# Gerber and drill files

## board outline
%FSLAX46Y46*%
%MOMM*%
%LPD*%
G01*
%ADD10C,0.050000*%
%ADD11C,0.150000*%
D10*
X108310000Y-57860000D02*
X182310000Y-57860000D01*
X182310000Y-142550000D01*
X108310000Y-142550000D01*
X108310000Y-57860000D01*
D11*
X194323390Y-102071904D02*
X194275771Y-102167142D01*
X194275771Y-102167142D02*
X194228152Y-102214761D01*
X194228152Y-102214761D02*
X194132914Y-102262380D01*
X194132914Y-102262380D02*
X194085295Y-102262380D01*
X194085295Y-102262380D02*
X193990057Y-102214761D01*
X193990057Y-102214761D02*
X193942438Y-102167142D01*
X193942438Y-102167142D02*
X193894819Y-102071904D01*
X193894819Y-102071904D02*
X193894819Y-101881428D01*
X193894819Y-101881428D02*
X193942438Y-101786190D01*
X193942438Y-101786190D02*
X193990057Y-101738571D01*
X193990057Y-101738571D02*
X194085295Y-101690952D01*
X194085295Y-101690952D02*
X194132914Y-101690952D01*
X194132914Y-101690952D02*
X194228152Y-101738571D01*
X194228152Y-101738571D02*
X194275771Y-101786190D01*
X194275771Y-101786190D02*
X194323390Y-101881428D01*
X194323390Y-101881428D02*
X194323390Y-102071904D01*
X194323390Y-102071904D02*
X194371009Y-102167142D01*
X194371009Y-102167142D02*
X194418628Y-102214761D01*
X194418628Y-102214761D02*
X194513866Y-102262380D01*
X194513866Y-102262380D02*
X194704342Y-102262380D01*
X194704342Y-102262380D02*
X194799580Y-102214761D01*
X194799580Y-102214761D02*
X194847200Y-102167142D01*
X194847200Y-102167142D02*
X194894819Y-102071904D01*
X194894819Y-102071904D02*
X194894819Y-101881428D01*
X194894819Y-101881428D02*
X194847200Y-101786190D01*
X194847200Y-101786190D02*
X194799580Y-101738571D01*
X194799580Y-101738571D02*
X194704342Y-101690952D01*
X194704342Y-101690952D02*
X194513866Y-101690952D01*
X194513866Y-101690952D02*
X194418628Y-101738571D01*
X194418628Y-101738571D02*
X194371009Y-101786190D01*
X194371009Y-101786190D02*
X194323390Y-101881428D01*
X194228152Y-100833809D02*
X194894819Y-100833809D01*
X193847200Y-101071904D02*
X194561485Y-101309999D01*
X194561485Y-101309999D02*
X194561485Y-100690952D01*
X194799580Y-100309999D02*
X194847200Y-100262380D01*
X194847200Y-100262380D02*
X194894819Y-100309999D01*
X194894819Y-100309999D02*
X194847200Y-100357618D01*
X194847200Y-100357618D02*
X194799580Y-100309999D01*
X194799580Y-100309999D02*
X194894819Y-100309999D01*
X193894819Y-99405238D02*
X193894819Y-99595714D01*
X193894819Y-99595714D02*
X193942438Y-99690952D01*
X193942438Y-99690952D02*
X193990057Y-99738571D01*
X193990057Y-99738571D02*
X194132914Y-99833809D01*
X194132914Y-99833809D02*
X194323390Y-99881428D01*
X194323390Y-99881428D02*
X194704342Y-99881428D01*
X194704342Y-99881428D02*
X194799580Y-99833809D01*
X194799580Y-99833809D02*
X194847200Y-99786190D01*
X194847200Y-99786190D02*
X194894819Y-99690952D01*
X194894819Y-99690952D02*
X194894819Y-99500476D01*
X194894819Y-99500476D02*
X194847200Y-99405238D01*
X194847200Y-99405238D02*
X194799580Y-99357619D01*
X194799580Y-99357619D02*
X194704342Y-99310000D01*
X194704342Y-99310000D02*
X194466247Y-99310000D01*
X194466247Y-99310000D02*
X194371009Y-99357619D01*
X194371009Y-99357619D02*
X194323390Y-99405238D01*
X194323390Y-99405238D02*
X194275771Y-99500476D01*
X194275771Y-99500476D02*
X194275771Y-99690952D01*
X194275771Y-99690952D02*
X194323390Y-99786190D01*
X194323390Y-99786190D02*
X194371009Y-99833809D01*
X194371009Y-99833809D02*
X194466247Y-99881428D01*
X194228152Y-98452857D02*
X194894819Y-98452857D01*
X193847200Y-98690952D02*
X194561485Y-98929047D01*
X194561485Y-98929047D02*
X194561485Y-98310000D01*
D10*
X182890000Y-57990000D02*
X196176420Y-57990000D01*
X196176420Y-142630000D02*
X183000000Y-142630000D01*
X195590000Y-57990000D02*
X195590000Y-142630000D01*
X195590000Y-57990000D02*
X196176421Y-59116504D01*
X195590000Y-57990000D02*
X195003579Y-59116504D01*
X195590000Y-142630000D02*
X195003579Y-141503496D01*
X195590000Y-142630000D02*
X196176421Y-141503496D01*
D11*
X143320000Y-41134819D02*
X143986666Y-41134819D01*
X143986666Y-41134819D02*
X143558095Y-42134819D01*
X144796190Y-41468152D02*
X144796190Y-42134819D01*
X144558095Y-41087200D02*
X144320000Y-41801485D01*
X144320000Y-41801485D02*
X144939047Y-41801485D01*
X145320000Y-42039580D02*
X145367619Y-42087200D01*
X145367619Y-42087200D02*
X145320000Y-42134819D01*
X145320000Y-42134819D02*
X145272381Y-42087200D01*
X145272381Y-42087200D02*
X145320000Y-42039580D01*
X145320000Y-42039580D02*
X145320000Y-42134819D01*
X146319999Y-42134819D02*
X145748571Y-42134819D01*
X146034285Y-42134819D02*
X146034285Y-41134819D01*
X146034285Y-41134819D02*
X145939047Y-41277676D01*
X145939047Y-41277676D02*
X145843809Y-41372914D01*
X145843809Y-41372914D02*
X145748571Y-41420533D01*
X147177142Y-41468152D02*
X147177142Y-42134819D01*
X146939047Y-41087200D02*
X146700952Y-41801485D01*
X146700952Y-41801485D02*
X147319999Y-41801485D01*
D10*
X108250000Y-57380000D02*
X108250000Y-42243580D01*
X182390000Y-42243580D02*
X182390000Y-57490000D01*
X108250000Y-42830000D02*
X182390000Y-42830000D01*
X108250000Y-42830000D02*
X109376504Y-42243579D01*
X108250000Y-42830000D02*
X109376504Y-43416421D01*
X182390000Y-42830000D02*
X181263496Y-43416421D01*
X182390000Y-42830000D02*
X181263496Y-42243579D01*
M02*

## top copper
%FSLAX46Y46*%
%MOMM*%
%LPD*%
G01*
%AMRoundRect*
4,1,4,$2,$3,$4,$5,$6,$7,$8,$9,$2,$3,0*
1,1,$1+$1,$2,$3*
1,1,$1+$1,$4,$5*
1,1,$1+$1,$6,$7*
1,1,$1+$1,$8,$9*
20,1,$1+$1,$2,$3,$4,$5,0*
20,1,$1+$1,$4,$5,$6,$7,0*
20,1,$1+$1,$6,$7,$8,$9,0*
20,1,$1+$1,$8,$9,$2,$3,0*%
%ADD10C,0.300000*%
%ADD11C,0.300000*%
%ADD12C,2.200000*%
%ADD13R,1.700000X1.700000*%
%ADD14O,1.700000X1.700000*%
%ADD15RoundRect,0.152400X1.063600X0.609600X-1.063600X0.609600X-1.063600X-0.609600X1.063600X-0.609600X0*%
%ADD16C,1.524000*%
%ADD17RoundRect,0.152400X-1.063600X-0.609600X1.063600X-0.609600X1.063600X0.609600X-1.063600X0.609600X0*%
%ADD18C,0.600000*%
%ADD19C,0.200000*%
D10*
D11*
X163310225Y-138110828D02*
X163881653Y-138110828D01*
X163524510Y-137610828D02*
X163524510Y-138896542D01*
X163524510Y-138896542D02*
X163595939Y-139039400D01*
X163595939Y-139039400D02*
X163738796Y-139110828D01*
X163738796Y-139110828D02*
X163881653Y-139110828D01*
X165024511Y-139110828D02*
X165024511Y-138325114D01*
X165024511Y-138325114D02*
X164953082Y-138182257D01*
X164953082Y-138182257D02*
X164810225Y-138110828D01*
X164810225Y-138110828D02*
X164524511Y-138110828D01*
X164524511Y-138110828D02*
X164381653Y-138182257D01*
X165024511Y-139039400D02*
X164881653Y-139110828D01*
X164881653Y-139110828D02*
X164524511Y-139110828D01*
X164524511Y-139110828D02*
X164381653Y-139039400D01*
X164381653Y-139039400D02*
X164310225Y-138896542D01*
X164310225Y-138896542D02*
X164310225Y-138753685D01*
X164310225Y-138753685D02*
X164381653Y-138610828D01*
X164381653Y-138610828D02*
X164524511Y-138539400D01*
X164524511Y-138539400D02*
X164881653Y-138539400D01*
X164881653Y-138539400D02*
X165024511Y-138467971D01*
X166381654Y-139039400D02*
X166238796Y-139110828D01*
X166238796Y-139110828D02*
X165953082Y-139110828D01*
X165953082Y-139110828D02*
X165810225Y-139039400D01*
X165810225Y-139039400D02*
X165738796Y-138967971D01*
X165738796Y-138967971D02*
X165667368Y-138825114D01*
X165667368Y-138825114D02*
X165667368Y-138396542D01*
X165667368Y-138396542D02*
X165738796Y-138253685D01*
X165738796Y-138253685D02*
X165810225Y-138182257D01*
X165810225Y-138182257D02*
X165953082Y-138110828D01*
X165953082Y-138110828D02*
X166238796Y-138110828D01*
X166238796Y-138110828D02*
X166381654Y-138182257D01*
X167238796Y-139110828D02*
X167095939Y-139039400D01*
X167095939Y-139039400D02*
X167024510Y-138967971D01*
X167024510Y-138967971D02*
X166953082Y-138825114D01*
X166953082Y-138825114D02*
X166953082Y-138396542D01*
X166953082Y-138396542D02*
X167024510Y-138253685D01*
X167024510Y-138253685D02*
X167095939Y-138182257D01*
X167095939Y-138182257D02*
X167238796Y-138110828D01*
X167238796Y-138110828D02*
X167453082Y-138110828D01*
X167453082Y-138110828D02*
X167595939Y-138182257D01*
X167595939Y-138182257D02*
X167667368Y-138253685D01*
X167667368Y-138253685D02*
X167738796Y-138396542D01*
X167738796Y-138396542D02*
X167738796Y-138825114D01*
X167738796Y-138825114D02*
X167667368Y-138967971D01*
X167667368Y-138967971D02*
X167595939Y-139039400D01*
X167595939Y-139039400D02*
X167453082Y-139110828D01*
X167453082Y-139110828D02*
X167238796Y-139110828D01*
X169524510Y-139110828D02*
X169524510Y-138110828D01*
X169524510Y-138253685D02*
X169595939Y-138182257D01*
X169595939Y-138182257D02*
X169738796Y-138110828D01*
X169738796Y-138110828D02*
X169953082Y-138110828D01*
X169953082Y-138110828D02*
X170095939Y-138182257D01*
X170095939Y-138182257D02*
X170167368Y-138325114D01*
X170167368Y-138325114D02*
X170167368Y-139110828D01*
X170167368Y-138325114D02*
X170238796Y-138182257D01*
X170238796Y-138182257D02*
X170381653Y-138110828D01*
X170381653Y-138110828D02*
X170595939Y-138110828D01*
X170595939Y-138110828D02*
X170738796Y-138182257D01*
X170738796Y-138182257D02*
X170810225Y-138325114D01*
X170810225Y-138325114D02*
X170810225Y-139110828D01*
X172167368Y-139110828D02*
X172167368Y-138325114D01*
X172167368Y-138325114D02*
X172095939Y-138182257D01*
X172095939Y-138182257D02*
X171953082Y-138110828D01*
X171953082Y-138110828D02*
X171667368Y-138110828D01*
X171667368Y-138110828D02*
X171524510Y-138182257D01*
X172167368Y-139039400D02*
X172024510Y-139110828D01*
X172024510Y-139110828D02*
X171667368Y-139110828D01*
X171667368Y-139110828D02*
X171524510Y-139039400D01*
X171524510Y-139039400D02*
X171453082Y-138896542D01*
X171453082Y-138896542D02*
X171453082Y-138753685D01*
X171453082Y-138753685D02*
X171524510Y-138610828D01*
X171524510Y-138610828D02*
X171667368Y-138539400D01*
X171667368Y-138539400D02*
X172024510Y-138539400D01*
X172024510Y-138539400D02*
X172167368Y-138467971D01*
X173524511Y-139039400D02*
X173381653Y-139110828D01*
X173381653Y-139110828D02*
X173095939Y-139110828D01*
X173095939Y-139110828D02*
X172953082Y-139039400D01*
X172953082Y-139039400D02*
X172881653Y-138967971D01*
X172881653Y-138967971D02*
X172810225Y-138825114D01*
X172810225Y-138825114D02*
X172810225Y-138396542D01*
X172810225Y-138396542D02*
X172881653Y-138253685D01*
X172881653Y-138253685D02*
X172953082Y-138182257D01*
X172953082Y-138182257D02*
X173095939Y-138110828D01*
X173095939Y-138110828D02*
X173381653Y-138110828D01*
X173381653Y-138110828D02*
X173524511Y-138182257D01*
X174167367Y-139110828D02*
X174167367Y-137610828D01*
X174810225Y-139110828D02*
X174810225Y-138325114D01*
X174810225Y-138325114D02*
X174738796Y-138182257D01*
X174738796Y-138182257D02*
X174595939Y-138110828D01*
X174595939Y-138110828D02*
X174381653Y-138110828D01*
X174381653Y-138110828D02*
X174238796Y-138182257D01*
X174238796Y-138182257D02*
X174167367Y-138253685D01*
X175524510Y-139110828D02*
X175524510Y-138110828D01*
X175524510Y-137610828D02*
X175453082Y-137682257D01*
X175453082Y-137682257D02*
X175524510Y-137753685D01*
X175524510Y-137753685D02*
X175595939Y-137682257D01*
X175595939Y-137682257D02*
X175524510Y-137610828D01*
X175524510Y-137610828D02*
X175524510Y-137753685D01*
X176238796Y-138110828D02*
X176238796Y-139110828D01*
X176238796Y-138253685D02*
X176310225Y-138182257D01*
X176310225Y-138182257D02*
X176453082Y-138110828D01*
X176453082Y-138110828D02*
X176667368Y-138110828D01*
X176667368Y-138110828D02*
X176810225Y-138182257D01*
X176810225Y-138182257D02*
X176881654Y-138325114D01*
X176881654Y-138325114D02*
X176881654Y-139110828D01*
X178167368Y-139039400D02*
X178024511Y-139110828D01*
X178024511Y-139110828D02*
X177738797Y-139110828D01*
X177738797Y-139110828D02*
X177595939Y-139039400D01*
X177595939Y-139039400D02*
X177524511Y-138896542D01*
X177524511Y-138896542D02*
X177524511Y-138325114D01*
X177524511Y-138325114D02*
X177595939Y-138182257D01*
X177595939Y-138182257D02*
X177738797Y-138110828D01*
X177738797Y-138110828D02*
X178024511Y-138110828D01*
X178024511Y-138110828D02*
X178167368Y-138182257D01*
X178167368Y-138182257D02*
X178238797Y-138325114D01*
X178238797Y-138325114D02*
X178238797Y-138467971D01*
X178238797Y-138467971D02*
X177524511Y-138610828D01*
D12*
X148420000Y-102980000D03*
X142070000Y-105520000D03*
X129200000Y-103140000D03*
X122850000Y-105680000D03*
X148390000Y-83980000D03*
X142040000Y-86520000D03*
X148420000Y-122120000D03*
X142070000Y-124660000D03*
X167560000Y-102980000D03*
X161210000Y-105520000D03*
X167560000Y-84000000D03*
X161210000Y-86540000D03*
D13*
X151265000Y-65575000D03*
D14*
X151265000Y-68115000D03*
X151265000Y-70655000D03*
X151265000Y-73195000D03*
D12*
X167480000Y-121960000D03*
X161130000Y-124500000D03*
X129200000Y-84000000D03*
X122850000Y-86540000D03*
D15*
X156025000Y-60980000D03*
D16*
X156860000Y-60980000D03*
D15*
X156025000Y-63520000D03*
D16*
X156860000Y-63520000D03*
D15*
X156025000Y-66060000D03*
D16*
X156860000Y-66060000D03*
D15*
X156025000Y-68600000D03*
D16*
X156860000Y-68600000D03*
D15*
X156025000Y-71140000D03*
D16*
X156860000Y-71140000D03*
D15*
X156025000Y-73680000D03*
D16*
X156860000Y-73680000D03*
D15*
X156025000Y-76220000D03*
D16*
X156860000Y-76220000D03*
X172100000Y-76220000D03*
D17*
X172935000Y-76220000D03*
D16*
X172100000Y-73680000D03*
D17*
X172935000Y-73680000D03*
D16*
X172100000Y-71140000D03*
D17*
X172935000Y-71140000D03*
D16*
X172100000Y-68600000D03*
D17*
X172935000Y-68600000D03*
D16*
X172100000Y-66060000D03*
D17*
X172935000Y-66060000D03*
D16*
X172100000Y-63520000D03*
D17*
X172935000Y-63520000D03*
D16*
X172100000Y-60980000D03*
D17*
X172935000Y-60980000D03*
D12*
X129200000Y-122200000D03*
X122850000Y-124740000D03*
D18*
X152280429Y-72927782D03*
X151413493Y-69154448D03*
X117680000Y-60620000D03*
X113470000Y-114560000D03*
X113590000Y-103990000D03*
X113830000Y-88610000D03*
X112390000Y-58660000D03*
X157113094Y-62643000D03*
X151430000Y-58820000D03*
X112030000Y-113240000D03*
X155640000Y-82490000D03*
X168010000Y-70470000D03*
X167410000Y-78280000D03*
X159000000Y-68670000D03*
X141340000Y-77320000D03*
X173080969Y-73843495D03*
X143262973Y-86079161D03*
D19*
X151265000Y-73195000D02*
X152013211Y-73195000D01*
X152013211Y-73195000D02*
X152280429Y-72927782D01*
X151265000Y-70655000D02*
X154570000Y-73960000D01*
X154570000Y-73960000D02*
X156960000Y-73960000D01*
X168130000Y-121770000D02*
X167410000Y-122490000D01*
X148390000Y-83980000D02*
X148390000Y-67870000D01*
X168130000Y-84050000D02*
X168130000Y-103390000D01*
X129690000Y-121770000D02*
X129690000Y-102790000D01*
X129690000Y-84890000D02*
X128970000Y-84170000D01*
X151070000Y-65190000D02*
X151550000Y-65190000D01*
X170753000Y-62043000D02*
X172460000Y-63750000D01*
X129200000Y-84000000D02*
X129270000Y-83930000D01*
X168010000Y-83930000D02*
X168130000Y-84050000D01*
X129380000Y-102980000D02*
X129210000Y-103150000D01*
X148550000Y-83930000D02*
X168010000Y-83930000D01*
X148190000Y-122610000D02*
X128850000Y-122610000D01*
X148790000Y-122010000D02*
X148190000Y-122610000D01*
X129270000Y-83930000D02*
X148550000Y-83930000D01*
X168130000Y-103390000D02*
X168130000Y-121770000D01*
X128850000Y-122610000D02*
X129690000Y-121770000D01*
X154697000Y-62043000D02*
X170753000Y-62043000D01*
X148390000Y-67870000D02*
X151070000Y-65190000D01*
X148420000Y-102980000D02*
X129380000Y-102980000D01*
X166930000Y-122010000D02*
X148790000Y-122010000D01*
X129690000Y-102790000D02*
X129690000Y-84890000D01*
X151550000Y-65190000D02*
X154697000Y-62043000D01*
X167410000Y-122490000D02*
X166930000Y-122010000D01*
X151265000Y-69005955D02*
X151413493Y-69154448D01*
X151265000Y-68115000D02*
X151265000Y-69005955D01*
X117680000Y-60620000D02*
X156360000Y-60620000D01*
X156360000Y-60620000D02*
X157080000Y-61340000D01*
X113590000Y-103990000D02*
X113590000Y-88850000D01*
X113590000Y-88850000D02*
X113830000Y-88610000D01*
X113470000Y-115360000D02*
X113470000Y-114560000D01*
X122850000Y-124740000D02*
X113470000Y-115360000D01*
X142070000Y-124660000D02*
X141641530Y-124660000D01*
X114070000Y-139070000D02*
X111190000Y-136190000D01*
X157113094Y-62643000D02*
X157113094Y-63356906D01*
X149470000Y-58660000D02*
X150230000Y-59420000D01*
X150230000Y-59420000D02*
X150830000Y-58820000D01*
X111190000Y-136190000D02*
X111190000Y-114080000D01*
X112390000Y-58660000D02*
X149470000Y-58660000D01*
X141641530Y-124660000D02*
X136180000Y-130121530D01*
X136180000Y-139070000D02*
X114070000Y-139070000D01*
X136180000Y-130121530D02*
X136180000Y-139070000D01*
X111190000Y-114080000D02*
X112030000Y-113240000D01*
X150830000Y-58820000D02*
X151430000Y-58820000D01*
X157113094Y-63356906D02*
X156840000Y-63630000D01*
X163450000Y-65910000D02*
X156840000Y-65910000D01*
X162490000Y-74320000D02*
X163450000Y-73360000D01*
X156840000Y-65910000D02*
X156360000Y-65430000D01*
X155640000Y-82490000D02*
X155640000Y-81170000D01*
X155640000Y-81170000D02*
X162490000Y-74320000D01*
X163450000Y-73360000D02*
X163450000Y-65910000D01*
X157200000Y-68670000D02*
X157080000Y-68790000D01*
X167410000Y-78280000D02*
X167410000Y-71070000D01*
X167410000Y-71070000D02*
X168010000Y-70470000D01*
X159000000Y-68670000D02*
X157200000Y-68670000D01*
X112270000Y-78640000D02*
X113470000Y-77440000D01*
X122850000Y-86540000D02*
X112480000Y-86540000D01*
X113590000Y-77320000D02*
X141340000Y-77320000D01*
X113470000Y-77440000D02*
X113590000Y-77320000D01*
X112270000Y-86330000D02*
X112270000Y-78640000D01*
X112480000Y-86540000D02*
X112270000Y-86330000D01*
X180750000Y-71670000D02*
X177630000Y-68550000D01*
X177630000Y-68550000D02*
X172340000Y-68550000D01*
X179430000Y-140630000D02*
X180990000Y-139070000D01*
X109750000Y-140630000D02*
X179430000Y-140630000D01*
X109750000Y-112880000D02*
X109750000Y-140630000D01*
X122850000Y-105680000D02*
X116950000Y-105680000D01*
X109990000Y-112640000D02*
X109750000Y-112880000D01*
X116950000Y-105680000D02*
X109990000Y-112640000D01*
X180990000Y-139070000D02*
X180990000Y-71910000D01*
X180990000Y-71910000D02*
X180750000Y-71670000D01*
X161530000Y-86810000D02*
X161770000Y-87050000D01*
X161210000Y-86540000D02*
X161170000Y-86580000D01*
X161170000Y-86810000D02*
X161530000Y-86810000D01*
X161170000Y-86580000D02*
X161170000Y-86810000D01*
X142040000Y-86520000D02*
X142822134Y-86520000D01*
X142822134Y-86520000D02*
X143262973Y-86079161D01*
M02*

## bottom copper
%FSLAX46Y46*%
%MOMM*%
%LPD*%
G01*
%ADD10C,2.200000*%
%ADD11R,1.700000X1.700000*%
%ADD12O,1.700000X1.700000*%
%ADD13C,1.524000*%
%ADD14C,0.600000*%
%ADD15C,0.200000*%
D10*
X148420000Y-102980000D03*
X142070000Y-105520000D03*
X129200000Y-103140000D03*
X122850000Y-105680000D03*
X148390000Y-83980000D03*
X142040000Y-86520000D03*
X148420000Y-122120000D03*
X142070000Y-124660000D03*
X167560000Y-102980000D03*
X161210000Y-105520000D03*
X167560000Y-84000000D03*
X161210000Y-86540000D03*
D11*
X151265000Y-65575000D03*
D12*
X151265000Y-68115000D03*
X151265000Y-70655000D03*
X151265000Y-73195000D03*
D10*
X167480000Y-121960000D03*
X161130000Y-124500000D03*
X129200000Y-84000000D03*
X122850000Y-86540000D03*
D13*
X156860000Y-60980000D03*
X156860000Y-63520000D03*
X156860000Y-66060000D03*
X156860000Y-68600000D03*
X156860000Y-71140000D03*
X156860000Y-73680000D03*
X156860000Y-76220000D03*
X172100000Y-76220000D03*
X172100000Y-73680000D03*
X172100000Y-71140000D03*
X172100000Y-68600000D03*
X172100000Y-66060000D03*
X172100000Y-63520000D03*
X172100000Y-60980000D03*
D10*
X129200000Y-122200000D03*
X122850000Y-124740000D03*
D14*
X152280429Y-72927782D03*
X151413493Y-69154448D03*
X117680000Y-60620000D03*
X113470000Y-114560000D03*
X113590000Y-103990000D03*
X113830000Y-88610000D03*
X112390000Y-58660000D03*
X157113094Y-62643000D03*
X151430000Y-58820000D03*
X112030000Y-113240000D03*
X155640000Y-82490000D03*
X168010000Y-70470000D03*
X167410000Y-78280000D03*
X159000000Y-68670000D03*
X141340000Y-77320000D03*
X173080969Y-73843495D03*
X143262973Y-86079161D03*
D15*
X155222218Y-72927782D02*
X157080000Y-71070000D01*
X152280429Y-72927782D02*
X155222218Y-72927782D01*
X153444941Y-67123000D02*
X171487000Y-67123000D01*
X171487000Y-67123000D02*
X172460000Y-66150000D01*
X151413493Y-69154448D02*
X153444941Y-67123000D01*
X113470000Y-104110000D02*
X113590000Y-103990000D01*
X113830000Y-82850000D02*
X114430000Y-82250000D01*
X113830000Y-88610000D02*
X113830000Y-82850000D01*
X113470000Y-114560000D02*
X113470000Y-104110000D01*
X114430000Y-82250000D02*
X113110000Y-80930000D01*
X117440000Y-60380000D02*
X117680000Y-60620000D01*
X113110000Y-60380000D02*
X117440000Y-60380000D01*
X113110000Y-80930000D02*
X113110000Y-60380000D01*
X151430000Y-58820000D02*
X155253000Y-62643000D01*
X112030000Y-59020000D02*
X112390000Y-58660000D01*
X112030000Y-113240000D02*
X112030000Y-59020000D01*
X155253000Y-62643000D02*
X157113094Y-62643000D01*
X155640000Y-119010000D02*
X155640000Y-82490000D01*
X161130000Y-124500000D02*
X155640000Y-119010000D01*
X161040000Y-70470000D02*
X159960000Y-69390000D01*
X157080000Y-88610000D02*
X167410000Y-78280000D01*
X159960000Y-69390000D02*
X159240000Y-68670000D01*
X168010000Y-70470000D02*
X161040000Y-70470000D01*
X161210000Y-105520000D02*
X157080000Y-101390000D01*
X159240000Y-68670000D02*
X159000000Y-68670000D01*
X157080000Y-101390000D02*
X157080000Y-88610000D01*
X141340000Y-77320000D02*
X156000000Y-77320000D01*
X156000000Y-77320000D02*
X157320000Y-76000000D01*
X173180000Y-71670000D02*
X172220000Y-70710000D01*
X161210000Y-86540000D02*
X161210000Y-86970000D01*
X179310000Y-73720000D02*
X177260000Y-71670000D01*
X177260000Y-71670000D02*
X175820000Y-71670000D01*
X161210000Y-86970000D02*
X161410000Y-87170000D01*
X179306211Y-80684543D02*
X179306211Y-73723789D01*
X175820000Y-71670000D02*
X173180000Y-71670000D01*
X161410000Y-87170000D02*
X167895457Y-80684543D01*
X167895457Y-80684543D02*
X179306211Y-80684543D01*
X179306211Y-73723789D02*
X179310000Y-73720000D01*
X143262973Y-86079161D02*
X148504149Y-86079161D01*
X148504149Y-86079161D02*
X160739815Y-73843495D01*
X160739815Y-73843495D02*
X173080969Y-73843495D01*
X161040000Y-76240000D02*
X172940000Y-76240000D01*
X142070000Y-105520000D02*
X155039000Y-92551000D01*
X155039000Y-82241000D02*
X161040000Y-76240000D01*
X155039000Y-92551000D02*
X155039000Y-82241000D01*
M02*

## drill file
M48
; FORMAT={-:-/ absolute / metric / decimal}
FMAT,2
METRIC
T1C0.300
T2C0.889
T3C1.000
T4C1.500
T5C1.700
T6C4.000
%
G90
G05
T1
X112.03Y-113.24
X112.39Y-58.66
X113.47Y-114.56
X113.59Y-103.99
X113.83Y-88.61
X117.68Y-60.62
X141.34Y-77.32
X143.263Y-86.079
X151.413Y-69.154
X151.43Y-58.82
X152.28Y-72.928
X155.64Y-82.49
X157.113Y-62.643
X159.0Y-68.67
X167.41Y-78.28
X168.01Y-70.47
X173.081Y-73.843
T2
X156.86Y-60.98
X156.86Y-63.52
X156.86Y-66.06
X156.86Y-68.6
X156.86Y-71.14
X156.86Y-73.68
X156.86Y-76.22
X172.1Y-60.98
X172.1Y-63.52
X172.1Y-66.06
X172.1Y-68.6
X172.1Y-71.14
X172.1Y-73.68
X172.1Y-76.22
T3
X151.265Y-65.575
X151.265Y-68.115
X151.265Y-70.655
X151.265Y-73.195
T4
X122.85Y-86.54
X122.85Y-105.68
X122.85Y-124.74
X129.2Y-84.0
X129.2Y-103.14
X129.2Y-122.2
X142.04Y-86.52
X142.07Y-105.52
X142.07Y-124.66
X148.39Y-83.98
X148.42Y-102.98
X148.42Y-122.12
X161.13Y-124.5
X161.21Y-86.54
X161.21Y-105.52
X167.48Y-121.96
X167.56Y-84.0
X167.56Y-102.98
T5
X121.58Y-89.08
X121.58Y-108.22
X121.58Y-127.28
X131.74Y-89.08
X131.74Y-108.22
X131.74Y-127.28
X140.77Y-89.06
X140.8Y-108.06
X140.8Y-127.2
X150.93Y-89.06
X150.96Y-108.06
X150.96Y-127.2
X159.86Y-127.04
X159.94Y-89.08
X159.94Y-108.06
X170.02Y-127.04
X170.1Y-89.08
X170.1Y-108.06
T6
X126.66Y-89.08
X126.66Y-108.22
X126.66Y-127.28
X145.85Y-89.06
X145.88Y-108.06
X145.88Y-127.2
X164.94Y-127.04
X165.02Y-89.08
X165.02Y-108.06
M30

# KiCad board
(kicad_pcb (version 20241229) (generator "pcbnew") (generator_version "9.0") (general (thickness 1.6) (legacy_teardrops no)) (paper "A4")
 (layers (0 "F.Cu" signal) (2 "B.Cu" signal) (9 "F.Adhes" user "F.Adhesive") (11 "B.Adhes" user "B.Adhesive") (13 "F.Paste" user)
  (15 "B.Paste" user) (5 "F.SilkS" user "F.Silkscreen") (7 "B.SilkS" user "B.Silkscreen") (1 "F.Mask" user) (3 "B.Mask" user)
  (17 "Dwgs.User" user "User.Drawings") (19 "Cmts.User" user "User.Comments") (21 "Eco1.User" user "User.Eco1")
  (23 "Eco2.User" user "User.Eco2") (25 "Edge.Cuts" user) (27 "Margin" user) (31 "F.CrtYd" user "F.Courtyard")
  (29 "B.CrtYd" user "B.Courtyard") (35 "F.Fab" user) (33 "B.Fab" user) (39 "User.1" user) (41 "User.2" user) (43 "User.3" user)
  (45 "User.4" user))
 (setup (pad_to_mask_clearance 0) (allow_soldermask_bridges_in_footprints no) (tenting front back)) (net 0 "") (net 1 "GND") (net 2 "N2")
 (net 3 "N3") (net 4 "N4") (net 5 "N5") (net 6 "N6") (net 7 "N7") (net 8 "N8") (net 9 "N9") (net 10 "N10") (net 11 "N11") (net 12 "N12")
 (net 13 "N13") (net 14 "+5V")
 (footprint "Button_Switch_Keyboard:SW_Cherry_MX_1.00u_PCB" (layer "F.Cu") (at 148.42 102.98)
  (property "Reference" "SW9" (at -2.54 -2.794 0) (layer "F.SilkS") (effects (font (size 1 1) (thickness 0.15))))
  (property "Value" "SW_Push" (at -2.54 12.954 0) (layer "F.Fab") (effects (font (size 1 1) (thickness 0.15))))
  (pad "" np_thru_hole circle (at -7.62 5.08) (size 1.7 1.7) (drill 1.7) (layers "*.Cu" "*.Mask"))
  (pad "" np_thru_hole circle (at -2.54 5.08) (size 4 4) (drill 4) (layers "*.Cu" "*.Mask"))
  (pad "" np_thru_hole circle (at 2.54 5.08) (size 1.7 1.7) (drill 1.7) (layers "*.Cu" "*.Mask"))
  (pad "1" thru_hole circle (at 0 0) (size 2.2 2.2) (drill 1.5) (layers "*.Cu" "*.Mask") (remove_unused_layers no) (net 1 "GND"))
  (pad "2" thru_hole circle (at -6.35 2.54) (size 2.2 2.2) (drill 1.5) (layers "*.Cu" "*.Mask") (remove_unused_layers no) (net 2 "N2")))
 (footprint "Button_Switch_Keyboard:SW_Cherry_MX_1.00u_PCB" (layer "F.Cu") (at 129.2 103.14)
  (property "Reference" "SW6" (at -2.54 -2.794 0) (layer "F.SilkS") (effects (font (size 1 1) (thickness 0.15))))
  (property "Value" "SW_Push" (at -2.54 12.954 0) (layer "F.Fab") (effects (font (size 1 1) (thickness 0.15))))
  (pad "" np_thru_hole circle (at -7.62 5.08) (size 1.7 1.7) (drill 1.7) (layers "*.Cu" "*.Mask"))
  (pad "" np_thru_hole circle (at -2.54 5.08) (size 4 4) (drill 4) (layers "*.Cu" "*.Mask"))
  (pad "" np_thru_hole circle (at 2.54 5.08) (size 1.7 1.7) (drill 1.7) (layers "*.Cu" "*.Mask"))
  (pad "1" thru_hole circle (at 0 0) (size 2.2 2.2) (drill 1.5) (layers "*.Cu" "*.Mask") (remove_unused_layers no) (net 1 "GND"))
  (pad "2" thru_hole circle (at -6.35 2.54) (size 2.2 2.2) (drill 1.5) (layers "*.Cu" "*.Mask") (remove_unused_layers no) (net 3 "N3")))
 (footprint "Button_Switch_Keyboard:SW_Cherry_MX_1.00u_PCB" (layer "F.Cu") (at 148.39 83.98)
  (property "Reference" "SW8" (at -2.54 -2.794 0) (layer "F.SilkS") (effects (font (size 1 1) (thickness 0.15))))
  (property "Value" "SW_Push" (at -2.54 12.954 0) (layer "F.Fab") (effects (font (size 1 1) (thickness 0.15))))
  (pad "" np_thru_hole circle (at -7.62 5.08) (size 1.7 1.7) (drill 1.7) (layers "*.Cu" "*.Mask"))
  (pad "" np_thru_hole circle (at -2.54 5.08) (size 4 4) (drill 4) (layers "*.Cu" "*.Mask"))
  (pad "" np_thru_hole circle (at 2.54 5.08) (size 1.7 1.7) (drill 1.7) (layers "*.Cu" "*.Mask"))
  (pad "1" thru_hole circle (at 0 0) (size 2.2 2.2) (drill 1.5) (layers "*.Cu" "*.Mask") (remove_unused_layers no) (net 1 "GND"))
  (pad "2" thru_hole circle (at -6.35 2.54) (size 2.2 2.2) (drill 1.5) (layers "*.Cu" "*.Mask") (remove_unused_layers no) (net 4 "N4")))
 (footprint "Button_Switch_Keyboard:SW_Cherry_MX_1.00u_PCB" (layer "F.Cu") (at 148.42 122.12)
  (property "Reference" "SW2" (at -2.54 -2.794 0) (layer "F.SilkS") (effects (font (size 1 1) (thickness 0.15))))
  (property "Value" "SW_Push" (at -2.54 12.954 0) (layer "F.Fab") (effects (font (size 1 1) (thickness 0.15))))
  (pad "" np_thru_hole circle (at -7.62 5.08) (size 1.7 1.7) (drill 1.7) (layers "*.Cu" "*.Mask"))
  (pad "" np_thru_hole circle (at -2.54 5.08) (size 4 4) (drill 4) (layers "*.Cu" "*.Mask"))
  (pad "" np_thru_hole circle (at 2.54 5.08) (size 1.7 1.7) (drill 1.7) (layers "*.Cu" "*.Mask"))
  (pad "1" thru_hole circle (at 0 0) (size 2.2 2.2) (drill 1.5) (layers "*.Cu" "*.Mask") (remove_unused_layers no) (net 1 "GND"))
  (pad "2" thru_hole circle (at -6.35 2.54) (size 2.2 2.2) (drill 1.5) (layers "*.Cu" "*.Mask") (remove_unused_layers no) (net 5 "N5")))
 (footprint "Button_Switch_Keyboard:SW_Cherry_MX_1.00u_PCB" (layer "F.Cu") (at 167.56 102.98)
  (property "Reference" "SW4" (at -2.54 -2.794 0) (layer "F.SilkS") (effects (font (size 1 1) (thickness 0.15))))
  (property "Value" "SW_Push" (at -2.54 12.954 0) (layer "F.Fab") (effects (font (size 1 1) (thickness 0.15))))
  (pad "" np_thru_hole circle (at -7.62 5.08) (size 1.7 1.7) (drill 1.7) (layers "*.Cu" "*.Mask"))
  (pad "" np_thru_hole circle (at -2.54 5.08) (size 4 4) (drill 4) (layers "*.Cu" "*.Mask"))
  (pad "" np_thru_hole circle (at 2.54 5.08) (size 1.7 1.7) (drill 1.7) (layers "*.Cu" "*.Mask"))
  (pad "1" thru_hole circle (at 0 0) (size 2.2 2.2) (drill 1.5) (layers "*.Cu" "*.Mask") (remove_unused_layers no) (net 1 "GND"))
  (pad "2" thru_hole circle (at -6.35 2.54) (size 2.2 2.2) (drill 1.5) (layers "*.Cu" "*.Mask") (remove_unused_layers no) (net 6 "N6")))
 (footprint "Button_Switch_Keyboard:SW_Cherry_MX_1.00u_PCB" (layer "F.Cu") (at 167.56 84)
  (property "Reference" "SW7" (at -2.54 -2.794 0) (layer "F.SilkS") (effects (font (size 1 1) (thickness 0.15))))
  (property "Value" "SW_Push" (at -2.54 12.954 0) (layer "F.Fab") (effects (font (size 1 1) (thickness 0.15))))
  (pad "" np_thru_hole circle (at -7.62 5.08) (size 1.7 1.7) (drill 1.7) (layers "*.Cu" "*.Mask"))
  (pad "" np_thru_hole circle (at -2.54 5.08) (size 4 4) (drill 4) (layers "*.Cu" "*.Mask"))
  (pad "" np_thru_hole circle (at 2.54 5.08) (size 1.7 1.7) (drill 1.7) (layers "*.Cu" "*.Mask"))
  (pad "1" thru_hole circle (at 0 0) (size 2.2 2.2) (drill 1.5) (layers "*.Cu" "*.Mask") (remove_unused_layers no) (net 1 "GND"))
  (pad "2" thru_hole circle (at -6.35 2.54) (size 2.2 2.2) (drill 1.5) (layers "*.Cu" "*.Mask") (remove_unused_layers no) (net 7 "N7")))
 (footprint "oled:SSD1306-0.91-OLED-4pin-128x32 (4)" (layer "F.Cu") (at 114.765 63.385)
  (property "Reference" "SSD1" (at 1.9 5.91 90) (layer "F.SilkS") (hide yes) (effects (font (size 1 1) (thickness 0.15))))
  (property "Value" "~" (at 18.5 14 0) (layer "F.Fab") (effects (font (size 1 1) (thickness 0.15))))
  (pad "1" thru_hole rect (at 36.5 2.19) (size 1.7 1.7) (drill 1) (layers "*.Cu" "*.Mask") (remove_unused_layers no) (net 1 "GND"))
  (pad "2" thru_hole oval (at 36.5 4.73) (size 1.7 1.7) (drill 1) (layers "*.Cu" "*.Mask") (remove_unused_layers no) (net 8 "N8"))
  (pad "3" thru_hole oval (at 36.5 7.27) (size 1.7 1.7) (drill 1) (layers "*.Cu" "*.Mask") (remove_unused_layers no) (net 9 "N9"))
  (pad "4" thru_hole oval (at 36.5 9.81) (size 1.7 1.7) (drill 1) (layers "*.Cu" "*.Mask") (remove_unused_layers no) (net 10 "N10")))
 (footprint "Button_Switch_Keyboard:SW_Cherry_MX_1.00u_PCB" (layer "F.Cu") (at 167.48 121.96)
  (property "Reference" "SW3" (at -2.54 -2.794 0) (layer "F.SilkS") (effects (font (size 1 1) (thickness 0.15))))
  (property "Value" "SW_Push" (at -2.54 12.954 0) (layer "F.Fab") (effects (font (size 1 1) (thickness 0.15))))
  (pad "" np_thru_hole circle (at -7.62 5.08) (size 1.7 1.7) (drill 1.7) (layers "*.Cu" "*.Mask"))
  (pad "" np_thru_hole circle (at -2.54 5.08) (size 4 4) (drill 4) (layers "*.Cu" "*.Mask"))
  (pad "" np_thru_hole circle (at 2.54 5.08) (size 1.7 1.7) (drill 1.7) (layers "*.Cu" "*.Mask"))
  (pad "1" thru_hole circle (at 0 0) (size 2.2 2.2) (drill 1.5) (layers "*.Cu" "*.Mask") (remove_unused_layers no) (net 1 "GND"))
  (pad "2" thru_hole circle (at -6.35 2.54) (size 2.2 2.2) (drill 1.5) (layers "*.Cu" "*.Mask") (remove_unused_layers no) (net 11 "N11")))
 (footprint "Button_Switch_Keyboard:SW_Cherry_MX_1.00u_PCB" (layer "F.Cu") (at 129.2 84)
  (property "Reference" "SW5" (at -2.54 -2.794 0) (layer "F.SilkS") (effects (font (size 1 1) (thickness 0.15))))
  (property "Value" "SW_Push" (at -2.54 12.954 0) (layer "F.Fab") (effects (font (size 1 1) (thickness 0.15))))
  (pad "" np_thru_hole circle (at -7.62 5.08) (size 1.7 1.7) (drill 1.7) (layers "*.Cu" "*.Mask"))
  (pad "" np_thru_hole circle (at -2.54 5.08) (size 4 4) (drill 4) (layers "*.Cu" "*.Mask"))
  (pad "" np_thru_hole circle (at 2.54 5.08) (size 1.7 1.7) (drill 1.7) (layers "*.Cu" "*.Mask"))
  (pad "1" thru_hole circle (at 0 0) (size 2.2 2.2) (drill 1.5) (layers "*.Cu" "*.Mask") (remove_unused_layers no) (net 1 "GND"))
  (pad "2" thru_hole circle (at -6.35 2.54) (size 2.2 2.2) (drill 1.5) (layers "*.Cu" "*.Mask") (remove_unused_layers no) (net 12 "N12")))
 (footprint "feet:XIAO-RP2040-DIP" (layer "F.Cu") (at 164.48 68.6)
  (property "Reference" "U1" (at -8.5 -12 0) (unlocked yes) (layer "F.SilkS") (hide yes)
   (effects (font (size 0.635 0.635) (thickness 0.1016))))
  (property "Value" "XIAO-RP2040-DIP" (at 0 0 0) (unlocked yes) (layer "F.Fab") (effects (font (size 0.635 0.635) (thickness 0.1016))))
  (pad "1" smd roundrect (at -8.455 -7.62 180) (size 2.432 1.524) (layers "F.Cu" "F.Mask") (roundrect_rratio 0.1) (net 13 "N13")
   (thermal_bridge_angle 45))
  (pad "1" thru_hole circle (at -7.62 -7.62 180) (size 1.524 1.524) (drill 0.889) (layers "*.Cu" "*.Mask") (remove_unused_layers no)
   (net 13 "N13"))
  (pad "2" smd roundrect (at -8.455 -5.08 180) (size 2.432 1.524) (layers "F.Cu" "F.Mask") (roundrect_rratio 0.1) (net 5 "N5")
   (thermal_bridge_angle 45))
  (pad "2" thru_hole circle (at -7.62 -5.08 180) (size 1.524 1.524) (drill 0.889) (layers "*.Cu" "*.Mask") (remove_unused_layers no)
   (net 5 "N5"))
  (pad "3" smd roundrect (at -8.455 -2.54 180) (size 2.432 1.524) (layers "F.Cu" "F.Mask") (roundrect_rratio 0.1) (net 11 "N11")
   (thermal_bridge_angle 45))
  (pad "3" thru_hole circle (at -7.62 -2.54 180) (size 1.524 1.524) (drill 0.889) (layers "*.Cu" "*.Mask") (remove_unused_layers no)
   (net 11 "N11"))
  (pad "4" smd roundrect (at -8.455 0 180) (size 2.432 1.524) (layers "F.Cu" "F.Mask") (roundrect_rratio 0.1) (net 6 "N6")
   (thermal_bridge_angle 45))
  (pad "4" thru_hole circle (at -7.62 0 180) (size 1.524 1.524) (drill 0.889) (layers "*.Cu" "*.Mask") (remove_unused_layers no)
   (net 6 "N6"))
  (pad "5" smd roundrect (at -8.455 2.54 180) (size 2.432 1.524) (layers "F.Cu" "F.Mask") (roundrect_rratio 0.1) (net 10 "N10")
   (thermal_bridge_angle 45))
  (pad "5" thru_hole circle (at -7.62 2.54 180) (size 1.524 1.524) (drill 0.889) (layers "*.Cu" "*.Mask") (remove_unused_layers no)
   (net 10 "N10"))
  (pad "6" smd roundrect (at -8.455 5.08 180) (size 2.432 1.524) (layers "F.Cu" "F.Mask") (roundrect_rratio 0.1) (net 9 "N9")
   (thermal_bridge_angle 45))
  (pad "6" thru_hole circle (at -7.62 5.08 180) (size 1.524 1.524) (drill 0.889) (layers "*.Cu" "*.Mask") (remove_unused_layers no)
   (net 9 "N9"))
  (pad "7" smd roundrect (at -8.455 7.62 180) (size 2.432 1.524) (layers "F.Cu" "F.Mask") (roundrect_rratio 0.1) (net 12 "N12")
   (thermal_bridge_angle 45))
  (pad "7" thru_hole circle (at -7.62 7.62 180) (size 1.524 1.524) (drill 0.889) (layers "*.Cu" "*.Mask") (remove_unused_layers no)
   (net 12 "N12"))
  (pad "8" thru_hole circle (at 7.62 7.62) (size 1.524 1.524) (drill 0.889) (layers "*.Cu" "*.Mask") (remove_unused_layers no) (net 2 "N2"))
  (pad "8" smd roundrect (at 8.455 7.62) (size 2.432 1.524) (layers "F.Cu" "F.Mask") (roundrect_rratio 0.1) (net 2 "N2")
   (thermal_bridge_angle 45))
  (pad "9" thru_hole circle (at 7.62 5.08) (size 1.524 1.524) (drill 0.889) (layers "*.Cu" "*.Mask") (remove_unused_layers no) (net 4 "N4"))
  (pad "9" smd roundrect (at 8.455 5.08) (size 2.432 1.524) (layers "F.Cu" "F.Mask") (roundrect_rratio 0.1) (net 4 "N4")
   (thermal_bridge_angle 45))
  (pad "10" thru_hole circle (at 7.62 2.54) (size 1.524 1.524) (drill 0.889) (layers "*.Cu" "*.Mask") (remove_unused_layers no) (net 7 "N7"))
  (pad "10" smd roundrect (at 8.455 2.54) (size 2.432 1.524) (layers "F.Cu" "F.Mask") (roundrect_rratio 0.1) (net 7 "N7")
   (thermal_bridge_angle 45))
  (pad "11" thru_hole circle (at 7.62 0) (size 1.524 1.524) (drill 0.889) (layers "*.Cu" "*.Mask") (remove_unused_layers no) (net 3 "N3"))
  (pad "11" smd roundrect (at 8.455 0) (size 2.432 1.524) (layers "F.Cu" "F.Mask") (roundrect_rratio 0.1) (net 3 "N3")
   (thermal_bridge_angle 45))
  (pad "12" thru_hole circle (at 7.62 -2.54) (size 1.524 1.524) (drill 0.889) (layers "*.Cu" "*.Mask") (remove_unused_layers no)
   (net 8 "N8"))
  (pad "12" smd roundrect (at 8.455 -2.54) (size 2.432 1.524) (layers "F.Cu" "F.Mask") (roundrect_rratio 0.1) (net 8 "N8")
   (thermal_bridge_angle 45))
  (pad "13" thru_hole circle (at 7.62 -5.08) (size 1.524 1.524) (drill 0.889) (layers "*.Cu" "*.Mask") (remove_unused_layers no)
   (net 1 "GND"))
  (pad "13" smd roundrect (at 8.455 -5.08) (size 2.432 1.524) (layers "F.Cu" "F.Mask") (roundrect_rratio 0.1) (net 1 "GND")
   (thermal_bridge_angle 45))
  (pad "14" thru_hole circle (at 7.62 -7.62) (size 1.524 1.524) (drill 0.889) (layers "*.Cu" "*.Mask") (remove_unused_layers no)
   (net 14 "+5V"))
  (pad "14" smd roundrect (at 8.455 -7.62) (size 2.432 1.524) (layers "F.Cu" "F.Mask") (roundrect_rratio 0.1) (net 14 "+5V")
   (thermal_bridge_angle 45)))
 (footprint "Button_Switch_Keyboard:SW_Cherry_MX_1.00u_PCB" (layer "F.Cu") (at 129.2 122.2)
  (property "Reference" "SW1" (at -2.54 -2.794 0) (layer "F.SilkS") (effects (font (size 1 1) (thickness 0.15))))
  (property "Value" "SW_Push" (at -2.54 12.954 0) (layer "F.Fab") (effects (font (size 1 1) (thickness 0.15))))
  (pad "" np_thru_hole circle (at -7.62 5.08) (size 1.7 1.7) (drill 1.7) (layers "*.Cu" "*.Mask"))
  (pad "" np_thru_hole circle (at -2.54 5.08) (size 4 4) (drill 4) (layers "*.Cu" "*.Mask"))
  (pad "" np_thru_hole circle (at 2.54 5.08) (size 1.7 1.7) (drill 1.7) (layers "*.Cu" "*.Mask"))
  (pad "1" thru_hole circle (at 0 0) (size 2.2 2.2) (drill 1.5) (layers "*.Cu" "*.Mask") (remove_unused_layers no) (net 1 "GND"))
  (pad "2" thru_hole circle (at -6.35 2.54) (size 2.2 2.2) (drill 1.5) (layers "*.Cu" "*.Mask") (remove_unused_layers no) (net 13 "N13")))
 (gr_rect (start 108.31 57.86) (end 182.31 142.55) (stroke (width 0.05) (type default)) (fill no) (layer "Edge.Cuts"))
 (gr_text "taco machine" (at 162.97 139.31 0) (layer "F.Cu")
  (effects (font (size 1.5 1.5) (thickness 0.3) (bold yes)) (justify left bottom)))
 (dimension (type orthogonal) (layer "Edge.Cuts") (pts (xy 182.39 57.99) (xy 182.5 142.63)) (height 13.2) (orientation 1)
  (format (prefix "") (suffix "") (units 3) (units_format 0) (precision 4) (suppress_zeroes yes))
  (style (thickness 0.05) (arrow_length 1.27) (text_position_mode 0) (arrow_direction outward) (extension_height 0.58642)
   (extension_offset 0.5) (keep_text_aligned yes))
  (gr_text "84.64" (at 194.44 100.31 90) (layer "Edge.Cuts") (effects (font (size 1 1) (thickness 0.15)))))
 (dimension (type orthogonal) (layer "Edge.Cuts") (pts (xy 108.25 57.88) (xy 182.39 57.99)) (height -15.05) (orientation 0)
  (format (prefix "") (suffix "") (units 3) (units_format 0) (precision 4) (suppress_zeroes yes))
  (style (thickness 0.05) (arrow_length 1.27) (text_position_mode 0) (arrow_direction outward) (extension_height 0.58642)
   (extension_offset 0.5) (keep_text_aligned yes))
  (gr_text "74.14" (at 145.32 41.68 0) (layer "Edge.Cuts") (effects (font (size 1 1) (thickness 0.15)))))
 (segment (start 151.265 73.195) (end 152.013211 73.195) (width 0.2) (layer "F.Cu") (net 10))
 (segment (start 152.013211 73.195) (end 152.280429 72.927782) (width 0.2) (layer "F.Cu") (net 10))
 (via (at 152.280429 72.927782) (size 0.6) (drill 0.3) (layers "F.Cu" "B.Cu") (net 10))
 (segment (start 155.222218 72.927782) (end 157.08 71.07) (width 0.2) (layer "B.Cu") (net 10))
 (segment (start 152.280429 72.927782) (end 155.222218 72.927782) (width 0.2) (layer "B.Cu") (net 10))
 (segment (start 151.265 70.655) (end 154.57 73.96) (width 0.2) (layer "F.Cu") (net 9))
 (segment (start 154.57 73.96) (end 156.96 73.96) (width 0.2) (layer "F.Cu") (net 9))
 (segment (start 168.13 121.77) (end 167.41 122.49) (width 0.2) (layer "F.Cu") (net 1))
 (segment (start 148.39 83.98) (end 148.39 67.87) (width 0.2) (layer "F.Cu") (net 1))
 (segment (start 168.13 84.05) (end 168.13 103.39) (width 0.2) (layer "F.Cu") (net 1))
 (segment (start 129.69 121.77) (end 129.69 102.79) (width 0.2) (layer "F.Cu") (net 1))
 (segment (start 129.69 84.89) (end 128.97 84.17) (width 0.2) (layer "F.Cu") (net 1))
 (segment (start 151.07 65.19) (end 151.55 65.19) (width 0.2) (layer "F.Cu") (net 1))
 (segment (start 170.753 62.043) (end 172.46 63.75) (width 0.2) (layer "F.Cu") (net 1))
 (segment (start 129.2 84) (end 129.27 83.93) (width 0.2) (layer "F.Cu") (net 1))
 (segment (start 168.01 83.93) (end 168.13 84.05) (width 0.2) (layer "F.Cu") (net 1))
 (segment (start 129.38 102.98) (end 129.21 103.15) (width 0.2) (layer "F.Cu") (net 1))
 (segment (start 148.55 83.93) (end 168.01 83.93) (width 0.2) (layer "F.Cu") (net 1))
 (segment (start 148.19 122.61) (end 128.85 122.61) (width 0.2) (layer "F.Cu") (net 1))
 (segment (start 148.79 122.01) (end 148.19 122.61) (width 0.2) (layer "F.Cu") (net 1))
 (segment (start 129.27 83.93) (end 148.55 83.93) (width 0.2) (layer "F.Cu") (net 1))
 (segment (start 168.13 103.39) (end 168.13 121.77) (width 0.2) (layer "F.Cu") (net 1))
 (segment (start 128.85 122.61) (end 129.69 121.77) (width 0.2) (layer "F.Cu") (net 1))
 (segment (start 154.697 62.043) (end 170.753 62.043) (width 0.2) (layer "F.Cu") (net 1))
 (segment (start 148.39 67.87) (end 151.07 65.19) (width 0.2) (layer "F.Cu") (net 1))
 (segment (start 148.42 102.98) (end 129.38 102.98) (width 0.2) (layer "F.Cu") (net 1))
 (segment (start 166.93 122.01) (end 148.79 122.01) (width 0.2) (layer "F.Cu") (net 1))
 (segment (start 129.69 102.79) (end 129.69 84.89) (width 0.2) (layer "F.Cu") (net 1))
 (segment (start 151.55 65.19) (end 154.697 62.043) (width 0.2) (layer "F.Cu") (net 1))
 (segment (start 167.41 122.49) (end 166.93 122.01) (width 0.2) (layer "F.Cu") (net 1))
 (segment (start 151.265 69.005955) (end 151.413493 69.154448) (width 0.2) (layer "F.Cu") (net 8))
 (segment (start 151.265 68.115) (end 151.265 69.005955) (width 0.2) (layer "F.Cu") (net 8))
 (via (at 151.413493 69.154448) (size 0.6) (drill 0.3) (layers "F.Cu" "B.Cu") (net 8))
 (segment (start 153.444941 67.123) (end 171.487 67.123) (width 0.2) (layer "B.Cu") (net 8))
 (segment (start 171.487 67.123) (end 172.46 66.15) (width 0.2) (layer "B.Cu") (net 8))
 (segment (start 151.413493 69.154448) (end 153.444941 67.123) (width 0.2) (layer "B.Cu") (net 8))
 (segment (start 117.68 60.62) (end 156.36 60.62) (width 0.2) (layer "F.Cu") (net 13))
 (segment (start 156.36 60.62) (end 157.08 61.34) (width 0.2) (layer "F.Cu") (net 13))
 (segment (start 113.59 103.99) (end 113.59 88.85) (width 0.2) (layer "F.Cu") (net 13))
 (segment (start 113.59 88.85) (end 113.83 88.61) (width 0.2) (layer "F.Cu") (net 13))
 (segment (start 113.47 115.36) (end 113.47 114.56) (width 0.2) (layer "F.Cu") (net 13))
 (segment (start 122.85 124.74) (end 113.47 115.36) (width 0.2) (layer "F.Cu") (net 13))
 (via (at 117.68 60.62) (size 0.6) (drill 0.3) (layers "F.Cu" "B.Cu") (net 13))
 (via (at 113.47 114.56) (size 0.6) (drill 0.3) (layers "F.Cu" "B.Cu") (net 13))
 (via (at 113.59 103.99) (size 0.6) (drill 0.3) (layers "F.Cu" "B.Cu") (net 13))
 (via (at 113.83 88.61) (size 0.6) (drill 0.3) (layers "F.Cu" "B.Cu") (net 13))
 (segment (start 113.47 104.11) (end 113.59 103.99) (width 0.2) (layer "B.Cu") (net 13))
 (segment (start 113.83 82.85) (end 114.43 82.25) (width 0.2) (layer "B.Cu") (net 13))
 (segment (start 113.83 88.61) (end 113.83 82.85) (width 0.2) (layer "B.Cu") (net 13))
 (segment (start 113.47 114.56) (end 113.47 104.11) (width 0.2) (layer "B.Cu") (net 13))
 (segment (start 114.43 82.25) (end 113.11 80.93) (width 0.2) (layer "B.Cu") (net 13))
 (segment (start 117.44 60.38) (end 117.68 60.62) (width 0.2) (layer "B.Cu") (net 13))
 (segment (start 113.11 60.38) (end 117.44 60.38) (width 0.2) (layer "B.Cu") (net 13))
 (segment (start 113.11 80.93) (end 113.11 60.38) (width 0.2) (layer "B.Cu") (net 13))
 (segment (start 142.07 124.66) (end 141.64153 124.66) (width 0.2) (layer "F.Cu") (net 5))
 (segment (start 114.07 139.07) (end 111.19 136.19) (width 0.2) (layer "F.Cu") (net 5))
 (segment (start 157.113094 62.643) (end 157.113094 63.356906) (width 0.2) (layer "F.Cu") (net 5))
 (segment (start 149.47 58.66) (end 150.23 59.42) (width 0.2) (layer "F.Cu") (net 5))
 (segment (start 150.23 59.42) (end 150.83 58.82) (width 0.2) (layer "F.Cu") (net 5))
 (segment (start 111.19 136.19) (end 111.19 114.08) (width 0.2) (layer "F.Cu") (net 5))
 (segment (start 112.39 58.66) (end 149.47 58.66) (width 0.2) (layer "F.Cu") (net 5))
 (segment (start 141.64153 124.66) (end 136.18 130.12153) (width 0.2) (layer "F.Cu") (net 5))
 (segment (start 136.18 139.07) (end 114.07 139.07) (width 0.2) (layer "F.Cu") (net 5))
 (segment (start 136.18 130.12153) (end 136.18 139.07) (width 0.2) (layer "F.Cu") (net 5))
 (segment (start 111.19 114.08) (end 112.03 113.24) (width 0.2) (layer "F.Cu") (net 5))
 (segment (start 150.83 58.82) (end 151.43 58.82) (width 0.2) (layer "F.Cu") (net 5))
 (segment (start 157.113094 63.356906) (end 156.84 63.63) (width 0.2) (layer "F.Cu") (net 5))
 (via (at 112.39 58.66) (size 0.6) (drill 0.3) (layers "F.Cu" "B.Cu") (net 5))
 (via (at 157.113094 62.643) (size 0.6) (drill 0.3) (layers "F.Cu" "B.Cu") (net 5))
 (via (at 151.43 58.82) (size 0.6) (drill 0.3) (layers "F.Cu" "B.Cu") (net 5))
 (via (at 112.03 113.24) (size 0.6) (drill 0.3) (layers "F.Cu" "B.Cu") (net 5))
 (segment (start 151.43 58.82) (end 155.253 62.643) (width 0.2) (layer "B.Cu") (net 5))
 (segment (start 112.03 59.02) (end 112.39 58.66) (width 0.2) (layer "B.Cu") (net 5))
 (segment (start 112.03 113.24) (end 112.03 59.02) (width 0.2) (layer "B.Cu") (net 5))
 (segment (start 155.253 62.643) (end 157.113094 62.643) (width 0.2) (layer "B.Cu") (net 5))
 (segment (start 163.45 65.91) (end 156.84 65.91) (width 0.2) (layer "F.Cu") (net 11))
 (segment (start 162.49 74.32) (end 163.45 73.36) (width 0.2) (layer "F.Cu") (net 11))
 (segment (start 156.84 65.91) (end 156.36 65.43) (width 0.2) (layer "F.Cu") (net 11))
 (segment (start 155.64 82.49) (end 155.64 81.17) (width 0.2) (layer "F.Cu") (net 11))
 (segment (start 155.64 81.17) (end 162.49 74.32) (width 0.2) (layer "F.Cu") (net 11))
 (segment (start 163.45 73.36) (end 163.45 65.91) (width 0.2) (layer "F.Cu") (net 11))
 (via (at 155.64 82.49) (size 0.6) (drill 0.3) (layers "F.Cu" "B.Cu") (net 11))
 (segment (start 155.64 119.01) (end 155.64 82.49) (width 0.2) (layer "B.Cu") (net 11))
 (segment (start 161.13 124.5) (end 155.64 119.01) (width 0.2) (layer "B.Cu") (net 11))
 (segment (start 157.2 68.67) (end 157.08 68.79) (width 0.2) (layer "F.Cu") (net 6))
 (segment (start 167.41 78.28) (end 167.41 71.07) (width 0.2) (layer "F.Cu") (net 6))
 (segment (start 167.41 71.07) (end 168.01 70.47) (width 0.2) (layer "F.Cu") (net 6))
 (segment (start 159 68.67) (end 157.2 68.67) (width 0.2) (layer "F.Cu") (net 6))
 (via (at 168.01 70.47) (size 0.6) (drill 0.3) (layers "F.Cu" "B.Cu") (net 6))
 (via (at 167.41 78.28) (size 0.6) (drill 0.3) (layers "F.Cu" "B.Cu") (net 6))
 (via (at 159 68.67) (size 0.6) (drill 0.3) (layers "F.Cu" "B.Cu") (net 6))
 (segment (start 161.04 70.47) (end 159.96 69.39) (width 0.2) (layer "B.Cu") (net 6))
 (segment (start 157.08 88.61) (end 167.41 78.28) (width 0.2) (layer "B.Cu") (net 6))
 (segment (start 159.96 69.39) (end 159.24 68.67) (width 0.2) (layer "B.Cu") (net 6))
 (segment (start 168.01 70.47) (end 161.04 70.47) (width 0.2) (layer "B.Cu") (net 6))
 (segment (start 161.21 105.52) (end 157.08 101.39) (width 0.2) (layer "B.Cu") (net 6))
 (segment (start 159.24 68.67) (end 159 68.67) (width 0.2) (layer "B.Cu") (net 6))
 (segment (start 157.08 101.39) (end 157.08 88.61) (width 0.2) (layer "B.Cu") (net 6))
 (segment (start 112.27 78.64) (end 113.47 77.44) (width 0.2) (layer "F.Cu") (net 12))
 (segment (start 122.85 86.54) (end 112.48 86.54) (width 0.2) (layer "F.Cu") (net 12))
 (segment (start 113.59 77.32) (end 141.34 77.32) (width 0.2) (layer "F.Cu") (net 12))
 (segment (start 113.47 77.44) (end 113.59 77.32) (width 0.2) (layer "F.Cu") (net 12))
 (segment (start 112.27 86.33) (end 112.27 78.64) (width 0.2) (layer "F.Cu") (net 12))
 (segment (start 112.48 86.54) (end 112.27 86.33) (width 0.2) (layer "F.Cu") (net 12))
 (via (at 141.34 77.32) (size 0.6) (drill 0.3) (layers "F.Cu" "B.Cu") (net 12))
 (segment (start 141.34 77.32) (end 156 77.32) (width 0.2) (layer "B.Cu") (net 12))
 (segment (start 156 77.32) (end 157.32 76) (width 0.2) (layer "B.Cu") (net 12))
 (segment (start 180.75 71.67) (end 177.63 68.55) (width 0.2) (layer "F.Cu") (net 3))
 (segment (start 177.63 68.55) (end 172.34 68.55) (width 0.2) (layer "F.Cu") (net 3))
 (segment (start 179.43 140.63) (end 180.99 139.07) (width 0.2) (layer "F.Cu") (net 3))
 (segment (start 109.75 140.63) (end 179.43 140.63) (width 0.2) (layer "F.Cu") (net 3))
 (segment (start 109.75 112.88) (end 109.75 140.63) (width 0.2) (layer "F.Cu") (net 3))
 (segment (start 122.85 105.68) (end 116.95 105.68) (width 0.2) (layer "F.Cu") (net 3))
 (segment (start 109.99 112.64) (end 109.75 112.88) (width 0.2) (layer "F.Cu") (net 3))
 (segment (start 116.95 105.68) (end 109.99 112.64) (width 0.2) (layer "F.Cu") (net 3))
 (segment (start 180.99 139.07) (end 180.99 71.91) (width 0.2) (layer "F.Cu") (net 3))
 (segment (start 180.99 71.91) (end 180.75 71.67) (width 0.2) (layer "F.Cu") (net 3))
 (segment (start 161.53 86.81) (end 161.77 87.05) (width 0.2) (layer "F.Cu") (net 7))
 (segment (start 161.21 86.54) (end 161.17 86.58) (width 0.2) (layer "F.Cu") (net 7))
 (segment (start 161.17 86.81) (end 161.53 86.81) (width 0.2) (layer "F.Cu") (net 7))
 (segment (start 161.17 86.58) (end 161.17 86.81) (width 0.2) (layer "F.Cu") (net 7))
 (segment (start 173.18 71.67) (end 172.22 70.71) (width 0.2) (layer "B.Cu") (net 7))
 (segment (start 161.21 86.54) (end 161.21 86.97) (width 0.2) (layer "B.Cu") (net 7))
 (segment (start 179.31 73.72) (end 177.26 71.67) (width 0.2) (layer "B.Cu") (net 7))
 (segment (start 177.26 71.67) (end 175.82 71.67) (width 0.2) (layer "B.Cu") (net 7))
 (segment (start 161.21 86.97) (end 161.41 87.17) (width 0.2) (layer "B.Cu") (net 7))
 (segment (start 179.306211 80.684543) (end 179.306211 73.723789) (width 0.2) (layer "B.Cu") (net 7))
 (segment (start 175.82 71.67) (end 173.18 71.67) (width 0.2) (layer "B.Cu") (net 7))
 (segment (start 161.41 87.17) (end 167.895457 80.684543) (width 0.2) (layer "B.Cu") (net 7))
 (segment (start 167.895457 80.684543) (end 179.306211 80.684543) (width 0.2) (layer "B.Cu") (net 7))
 (segment (start 179.306211 73.723789) (end 179.31 73.72) (width 0.2) (layer "B.Cu") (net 7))
 (segment (start 142.04 86.52) (end 142.822134 86.52) (width 0.2) (layer "F.Cu") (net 4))
 (segment (start 142.822134 86.52) (end 143.262973 86.079161) (width 0.2) (layer "F.Cu") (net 4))
 (via (at 173.080969 73.843495) (size 0.6) (drill 0.3) (layers "F.Cu" "B.Cu") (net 4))
 (via (at 143.262973 86.079161) (size 0.6) (drill 0.3) (layers "F.Cu" "B.Cu") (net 4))
 (segment (start 143.262973 86.079161) (end 148.504149 86.079161) (width 0.2) (layer "B.Cu") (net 4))
 (segment (start 148.504149 86.079161) (end 160.739815 73.843495) (width 0.2) (layer "B.Cu") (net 4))
 (segment (start 160.739815 73.843495) (end 173.080969 73.843495) (width 0.2) (layer "B.Cu") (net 4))
 (segment (start 161.04 76.24) (end 172.94 76.24) (width 0.2) (layer "B.Cu") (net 2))
 (segment (start 142.07 105.52) (end 155.039 92.551) (width 0.2) (layer "B.Cu") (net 2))
 (segment (start 155.039 82.241) (end 161.04 76.24) (width 0.2) (layer "B.Cu") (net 2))
 (segment (start 155.039 92.551) (end 155.039 82.241) (width 0.2) (layer "B.Cu") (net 2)))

